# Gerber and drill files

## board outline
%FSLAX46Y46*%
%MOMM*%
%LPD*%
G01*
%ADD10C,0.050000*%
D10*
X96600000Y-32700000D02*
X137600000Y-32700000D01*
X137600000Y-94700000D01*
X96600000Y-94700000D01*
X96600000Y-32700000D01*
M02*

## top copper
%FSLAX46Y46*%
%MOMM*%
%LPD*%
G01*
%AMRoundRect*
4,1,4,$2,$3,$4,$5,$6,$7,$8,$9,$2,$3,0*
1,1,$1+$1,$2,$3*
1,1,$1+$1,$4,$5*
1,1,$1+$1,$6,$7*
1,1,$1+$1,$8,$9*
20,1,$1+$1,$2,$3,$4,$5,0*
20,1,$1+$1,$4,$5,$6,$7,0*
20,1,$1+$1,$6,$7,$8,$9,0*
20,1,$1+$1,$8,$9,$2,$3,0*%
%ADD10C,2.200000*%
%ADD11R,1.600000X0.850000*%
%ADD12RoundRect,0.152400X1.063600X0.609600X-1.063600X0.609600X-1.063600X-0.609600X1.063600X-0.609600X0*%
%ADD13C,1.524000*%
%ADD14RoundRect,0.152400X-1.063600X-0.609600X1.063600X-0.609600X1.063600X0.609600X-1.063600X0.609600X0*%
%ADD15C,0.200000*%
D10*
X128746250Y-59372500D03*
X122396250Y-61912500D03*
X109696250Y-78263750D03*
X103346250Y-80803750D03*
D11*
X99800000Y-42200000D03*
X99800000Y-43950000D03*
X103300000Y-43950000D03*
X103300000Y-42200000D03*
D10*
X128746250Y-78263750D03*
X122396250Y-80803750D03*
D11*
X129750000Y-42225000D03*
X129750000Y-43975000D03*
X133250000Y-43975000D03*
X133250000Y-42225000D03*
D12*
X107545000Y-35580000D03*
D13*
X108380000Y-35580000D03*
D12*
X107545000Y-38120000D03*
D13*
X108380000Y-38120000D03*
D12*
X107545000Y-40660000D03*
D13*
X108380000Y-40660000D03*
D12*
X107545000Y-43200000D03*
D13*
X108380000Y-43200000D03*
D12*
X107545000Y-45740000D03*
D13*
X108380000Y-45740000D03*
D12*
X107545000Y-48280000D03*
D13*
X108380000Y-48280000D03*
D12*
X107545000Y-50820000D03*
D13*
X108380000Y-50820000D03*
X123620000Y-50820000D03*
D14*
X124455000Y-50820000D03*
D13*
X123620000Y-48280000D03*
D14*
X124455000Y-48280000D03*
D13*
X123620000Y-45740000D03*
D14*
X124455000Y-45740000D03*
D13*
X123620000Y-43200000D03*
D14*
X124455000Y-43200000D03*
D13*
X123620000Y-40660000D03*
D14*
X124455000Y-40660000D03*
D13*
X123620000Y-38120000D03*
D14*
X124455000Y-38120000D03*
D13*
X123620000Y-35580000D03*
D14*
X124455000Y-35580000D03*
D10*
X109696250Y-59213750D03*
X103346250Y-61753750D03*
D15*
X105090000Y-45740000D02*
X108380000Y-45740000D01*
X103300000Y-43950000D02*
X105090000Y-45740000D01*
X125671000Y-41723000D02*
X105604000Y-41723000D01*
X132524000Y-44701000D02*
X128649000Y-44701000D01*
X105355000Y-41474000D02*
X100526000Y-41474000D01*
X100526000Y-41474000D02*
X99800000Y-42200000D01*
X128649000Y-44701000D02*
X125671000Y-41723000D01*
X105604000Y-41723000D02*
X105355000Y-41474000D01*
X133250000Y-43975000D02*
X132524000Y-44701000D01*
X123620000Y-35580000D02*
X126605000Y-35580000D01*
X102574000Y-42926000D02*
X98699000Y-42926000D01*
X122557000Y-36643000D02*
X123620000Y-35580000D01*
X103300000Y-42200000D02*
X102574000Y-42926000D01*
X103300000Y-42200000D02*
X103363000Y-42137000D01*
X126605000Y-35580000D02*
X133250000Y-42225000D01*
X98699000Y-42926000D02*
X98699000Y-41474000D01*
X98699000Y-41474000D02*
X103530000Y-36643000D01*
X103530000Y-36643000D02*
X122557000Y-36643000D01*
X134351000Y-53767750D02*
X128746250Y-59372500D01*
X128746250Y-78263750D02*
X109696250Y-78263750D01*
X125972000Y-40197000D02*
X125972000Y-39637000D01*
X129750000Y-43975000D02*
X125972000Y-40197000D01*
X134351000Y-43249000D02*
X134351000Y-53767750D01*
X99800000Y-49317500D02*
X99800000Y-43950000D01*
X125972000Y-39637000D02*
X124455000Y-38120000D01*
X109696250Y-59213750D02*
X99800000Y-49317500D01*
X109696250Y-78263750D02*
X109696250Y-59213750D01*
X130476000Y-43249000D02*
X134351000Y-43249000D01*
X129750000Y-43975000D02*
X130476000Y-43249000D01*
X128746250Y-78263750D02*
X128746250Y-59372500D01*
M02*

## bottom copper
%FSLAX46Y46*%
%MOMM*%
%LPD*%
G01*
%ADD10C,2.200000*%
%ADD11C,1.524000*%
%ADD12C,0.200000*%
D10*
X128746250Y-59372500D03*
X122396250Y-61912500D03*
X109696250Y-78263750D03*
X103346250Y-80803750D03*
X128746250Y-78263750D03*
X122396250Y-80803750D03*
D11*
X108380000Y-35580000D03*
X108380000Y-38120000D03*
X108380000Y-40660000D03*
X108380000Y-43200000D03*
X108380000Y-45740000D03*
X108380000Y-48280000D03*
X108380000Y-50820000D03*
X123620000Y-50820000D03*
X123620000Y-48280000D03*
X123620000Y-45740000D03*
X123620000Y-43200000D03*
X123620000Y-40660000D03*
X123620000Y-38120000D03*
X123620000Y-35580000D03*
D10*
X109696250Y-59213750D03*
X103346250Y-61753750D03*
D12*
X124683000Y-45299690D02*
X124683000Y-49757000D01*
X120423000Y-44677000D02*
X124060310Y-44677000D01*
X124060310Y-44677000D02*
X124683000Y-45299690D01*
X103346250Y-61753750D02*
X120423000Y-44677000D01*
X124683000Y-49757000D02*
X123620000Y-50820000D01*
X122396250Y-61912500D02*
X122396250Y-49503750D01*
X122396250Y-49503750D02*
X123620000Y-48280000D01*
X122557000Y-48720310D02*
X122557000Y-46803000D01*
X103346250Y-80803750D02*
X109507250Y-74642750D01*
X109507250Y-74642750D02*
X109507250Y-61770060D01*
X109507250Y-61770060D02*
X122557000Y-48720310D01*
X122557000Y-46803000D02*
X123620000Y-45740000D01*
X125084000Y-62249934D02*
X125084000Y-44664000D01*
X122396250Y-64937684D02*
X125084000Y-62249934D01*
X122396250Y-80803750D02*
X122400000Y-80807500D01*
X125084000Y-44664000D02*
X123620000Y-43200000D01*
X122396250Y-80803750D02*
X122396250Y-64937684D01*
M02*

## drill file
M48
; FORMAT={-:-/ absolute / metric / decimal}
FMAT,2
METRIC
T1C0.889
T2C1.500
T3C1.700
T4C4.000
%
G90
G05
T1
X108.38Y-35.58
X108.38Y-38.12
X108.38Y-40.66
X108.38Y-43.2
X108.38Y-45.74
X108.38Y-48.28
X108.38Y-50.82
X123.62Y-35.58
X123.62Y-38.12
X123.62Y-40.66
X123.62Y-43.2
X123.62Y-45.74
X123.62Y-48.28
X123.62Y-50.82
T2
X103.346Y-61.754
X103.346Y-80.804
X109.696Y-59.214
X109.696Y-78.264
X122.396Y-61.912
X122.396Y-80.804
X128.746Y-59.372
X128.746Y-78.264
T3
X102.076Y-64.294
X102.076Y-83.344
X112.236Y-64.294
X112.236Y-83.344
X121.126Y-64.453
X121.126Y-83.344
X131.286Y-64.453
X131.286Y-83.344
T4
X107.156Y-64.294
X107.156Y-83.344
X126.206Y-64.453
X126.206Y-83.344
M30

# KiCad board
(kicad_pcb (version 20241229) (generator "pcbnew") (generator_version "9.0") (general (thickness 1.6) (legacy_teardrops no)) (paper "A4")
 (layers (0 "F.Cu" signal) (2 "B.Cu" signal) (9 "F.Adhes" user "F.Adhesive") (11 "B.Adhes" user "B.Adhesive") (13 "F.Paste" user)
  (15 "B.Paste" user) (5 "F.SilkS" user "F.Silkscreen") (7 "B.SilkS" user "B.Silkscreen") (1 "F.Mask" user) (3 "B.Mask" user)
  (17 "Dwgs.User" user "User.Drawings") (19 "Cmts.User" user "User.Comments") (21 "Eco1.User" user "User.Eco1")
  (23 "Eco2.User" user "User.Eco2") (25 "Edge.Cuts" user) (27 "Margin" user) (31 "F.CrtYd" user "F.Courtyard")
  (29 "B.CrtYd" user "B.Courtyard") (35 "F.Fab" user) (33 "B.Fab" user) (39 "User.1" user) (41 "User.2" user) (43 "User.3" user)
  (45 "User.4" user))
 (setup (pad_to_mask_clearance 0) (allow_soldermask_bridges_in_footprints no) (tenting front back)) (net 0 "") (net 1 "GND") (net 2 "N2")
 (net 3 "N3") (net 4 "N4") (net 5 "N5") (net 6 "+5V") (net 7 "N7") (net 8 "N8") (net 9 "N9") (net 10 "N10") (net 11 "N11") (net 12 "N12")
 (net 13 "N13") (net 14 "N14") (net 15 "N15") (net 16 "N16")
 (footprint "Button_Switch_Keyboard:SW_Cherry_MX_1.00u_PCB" (layer "F.Cu") (at 128.74625 59.3725)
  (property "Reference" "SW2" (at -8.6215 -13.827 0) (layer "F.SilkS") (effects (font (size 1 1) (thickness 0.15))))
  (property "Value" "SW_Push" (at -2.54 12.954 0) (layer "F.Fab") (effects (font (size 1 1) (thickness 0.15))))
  (pad "" np_thru_hole circle (at -7.62 5.08) (size 1.7 1.7) (drill 1.7) (layers "*.Cu" "*.Mask"))
  (pad "" np_thru_hole circle (at -2.54 5.08) (size 4 4) (drill 4) (layers "*.Cu" "*.Mask"))
  (pad "" np_thru_hole circle (at 2.54 5.08) (size 1.7 1.7) (drill 1.7) (layers "*.Cu" "*.Mask"))
  (pad "1" thru_hole circle (at 0 0) (size 2.2 2.2) (drill 1.5) (layers "*.Cu" "*.Mask") (remove_unused_layers no) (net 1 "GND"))
  (pad "2" thru_hole circle (at -6.35 2.54) (size 2.2 2.2) (drill 1.5) (layers "*.Cu" "*.Mask") (remove_unused_layers no) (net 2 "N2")))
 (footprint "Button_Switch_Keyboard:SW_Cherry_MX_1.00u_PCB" (layer "F.Cu") (at 109.69625 78.26375)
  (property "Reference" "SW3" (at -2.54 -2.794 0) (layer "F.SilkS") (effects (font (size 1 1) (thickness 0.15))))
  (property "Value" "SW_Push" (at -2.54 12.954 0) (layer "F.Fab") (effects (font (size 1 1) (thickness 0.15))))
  (pad "" np_thru_hole circle (at -7.62 5.08) (size 1.7 1.7) (drill 1.7) (layers "*.Cu" "*.Mask"))
  (pad "" np_thru_hole circle (at -2.54 5.08) (size 4 4) (drill 4) (layers "*.Cu" "*.Mask"))
  (pad "" np_thru_hole circle (at 2.54 5.08) (size 1.7 1.7) (drill 1.7) (layers "*.Cu" "*.Mask"))
  (pad "1" thru_hole circle (at 0 0) (size 2.2 2.2) (drill 1.5) (layers "*.Cu" "*.Mask") (remove_unused_layers no) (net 1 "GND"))
  (pad "2" thru_hole circle (at -6.35 2.54) (size 2.2 2.2) (drill 1.5) (layers "*.Cu" "*.Mask") (remove_unused_layers no) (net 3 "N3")))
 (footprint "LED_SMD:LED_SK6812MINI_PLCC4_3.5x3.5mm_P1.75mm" (layer "F.Cu") (at 101.55 43.075)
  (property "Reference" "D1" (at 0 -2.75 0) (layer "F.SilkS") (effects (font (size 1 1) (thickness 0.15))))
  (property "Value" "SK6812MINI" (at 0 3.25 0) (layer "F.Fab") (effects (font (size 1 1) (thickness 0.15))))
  (pad "1" smd rect (at -1.75 -0.875) (size 1.6 0.85) (layers "F.Cu" "F.Mask" "F.Paste") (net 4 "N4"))
  (pad "2" smd rect (at -1.75 0.875) (size 1.6 0.85) (layers "F.Cu" "F.Mask" "F.Paste") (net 1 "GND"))
  (pad "3" smd rect (at 1.75 0.875) (size 1.6 0.85) (layers "F.Cu" "F.Mask" "F.Paste") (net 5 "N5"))
  (pad "4" smd rect (at 1.75 -0.875) (size 1.6 0.85) (layers "F.Cu" "F.Mask" "F.Paste") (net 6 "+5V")))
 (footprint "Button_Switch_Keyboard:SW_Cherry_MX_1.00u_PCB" (layer "F.Cu") (at 128.74625 78.26375)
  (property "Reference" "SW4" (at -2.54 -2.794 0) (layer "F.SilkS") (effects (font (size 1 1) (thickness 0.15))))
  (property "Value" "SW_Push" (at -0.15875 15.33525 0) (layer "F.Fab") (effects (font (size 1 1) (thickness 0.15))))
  (pad "" np_thru_hole circle (at -7.62 5.08) (size 1.7 1.7) (drill 1.7) (layers "*.Cu" "*.Mask"))
  (pad "" np_thru_hole circle (at -2.54 5.08) (size 4 4) (drill 4) (layers "*.Cu" "*.Mask"))
  (pad "" np_thru_hole circle (at 2.54 5.08) (size 1.7 1.7) (drill 1.7) (layers "*.Cu" "*.Mask"))
  (pad "1" thru_hole circle (at 0 0) (size 2.2 2.2) (drill 1.5) (layers "*.Cu" "*.Mask") (remove_unused_layers no) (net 1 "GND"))
  (pad "2" thru_hole circle (at -6.35 2.54) (size 2.2 2.2) (drill 1.5) (layers "*.Cu" "*.Mask") (remove_unused_layers no) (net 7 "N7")))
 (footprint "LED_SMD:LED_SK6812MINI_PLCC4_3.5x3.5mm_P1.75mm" (layer "F.Cu") (at 131.5 43.1)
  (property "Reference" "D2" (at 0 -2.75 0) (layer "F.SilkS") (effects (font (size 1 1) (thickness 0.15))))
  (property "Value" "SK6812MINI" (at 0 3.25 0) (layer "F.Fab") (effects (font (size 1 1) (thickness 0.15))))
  (pad "1" smd rect (at -1.75 -0.875) (size 1.6 0.85) (layers "F.Cu" "F.Mask" "F.Paste") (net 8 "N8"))
  (pad "2" smd rect (at -1.75 0.875) (size 1.6 0.85) (layers "F.Cu" "F.Mask" "F.Paste") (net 1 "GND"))
  (pad "3" smd rect (at 1.75 0.875) (size 1.6 0.85) (layers "F.Cu" "F.Mask" "F.Paste") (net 4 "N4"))
  (pad "4" smd rect (at 1.75 -0.875) (size 1.6 0.85) (layers "F.Cu" "F.Mask" "F.Paste") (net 6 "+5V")))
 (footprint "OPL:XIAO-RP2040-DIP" (layer "F.Cu") (at 116 43.2)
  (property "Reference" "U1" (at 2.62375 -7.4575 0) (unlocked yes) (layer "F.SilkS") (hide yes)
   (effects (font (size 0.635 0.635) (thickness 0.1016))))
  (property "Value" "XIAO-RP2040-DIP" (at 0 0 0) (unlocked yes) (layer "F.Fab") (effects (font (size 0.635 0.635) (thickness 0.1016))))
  (pad "1" smd roundrect (at -8.455 -7.62 180) (size 2.432 1.524) (layers "F.Cu" "F.Mask") (roundrect_rratio 0.1) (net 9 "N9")
   (thermal_bridge_angle 45))
  (pad "1" thru_hole circle (at -7.62 -7.62 180) (size 1.524 1.524) (drill 0.889) (layers "*.Cu" "*.Mask") (remove_unused_layers no)
   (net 9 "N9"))
  (pad "2" smd roundrect (at -8.455 -5.08 180) (size 2.432 1.524) (layers "F.Cu" "F.Mask") (roundrect_rratio 0.1) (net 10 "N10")
   (thermal_bridge_angle 45))
  (pad "2" thru_hole circle (at -7.62 -5.08 180) (size 1.524 1.524) (drill 0.889) (layers "*.Cu" "*.Mask") (remove_unused_layers no)
   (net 10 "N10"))
  (pad "3" smd roundrect (at -8.455 -2.54 180) (size 2.432 1.524) (layers "F.Cu" "F.Mask") (roundrect_rratio 0.1) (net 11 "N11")
   (thermal_bridge_angle 45))
  (pad "3" thru_hole circle (at -7.62 -2.54 180) (size 1.524 1.524) (drill 0.889) (layers "*.Cu" "*.Mask") (remove_unused_layers no)
   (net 11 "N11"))
  (pad "4" smd roundrect (at -8.455 0 180) (size 2.432 1.524) (layers "F.Cu" "F.Mask") (roundrect_rratio 0.1) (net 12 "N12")
   (thermal_bridge_angle 45))
  (pad "4" thru_hole circle (at -7.62 0 180) (size 1.524 1.524) (drill 0.889) (layers "*.Cu" "*.Mask") (remove_unused_layers no)
   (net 12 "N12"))
  (pad "5" smd roundrect (at -8.455 2.54 180) (size 2.432 1.524) (layers "F.Cu" "F.Mask") (roundrect_rratio 0.1) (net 5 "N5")
   (thermal_bridge_angle 45))
  (pad "5" thru_hole circle (at -7.62 2.54 180) (size 1.524 1.524) (drill 0.889) (layers "*.Cu" "*.Mask") (remove_unused_layers no)
   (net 5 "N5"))
  (pad "6" smd roundrect (at -8.455 5.08 180) (size 2.432 1.524) (layers "F.Cu" "F.Mask") (roundrect_rratio 0.1) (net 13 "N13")
   (thermal_bridge_angle 45))
  (pad "6" thru_hole circle (at -7.62 5.08 180) (size 1.524 1.524) (drill 0.889) (layers "*.Cu" "*.Mask") (remove_unused_layers no)
   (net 13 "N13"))
  (pad "7" smd roundrect (at -8.455 7.62 180) (size 2.432 1.524) (layers "F.Cu" "F.Mask") (roundrect_rratio 0.1) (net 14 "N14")
   (thermal_bridge_angle 45))
  (pad "7" thru_hole circle (at -7.62 7.62 180) (size 1.524 1.524) (drill 0.889) (layers "*.Cu" "*.Mask") (remove_unused_layers no)
   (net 14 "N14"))
  (pad "8" thru_hole circle (at 7.62 7.62) (size 1.524 1.524) (drill 0.889) (layers "*.Cu" "*.Mask") (remove_unused_layers no)
   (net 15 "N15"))
  (pad "8" smd roundrect (at 8.455 7.62) (size 2.432 1.524) (layers "F.Cu" "F.Mask") (roundrect_rratio 0.1) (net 15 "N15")
   (thermal_bridge_angle 45))
  (pad "9" thru_hole circle (at 7.62 5.08) (size 1.524 1.524) (drill 0.889) (layers "*.Cu" "*.Mask") (remove_unused_layers no) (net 2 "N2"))
  (pad "9" smd roundrect (at 8.455 5.08) (size 2.432 1.524) (layers "F.Cu" "F.Mask") (roundrect_rratio 0.1) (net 2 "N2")
   (thermal_bridge_angle 45))
  (pad "10" thru_hole circle (at 7.62 2.54) (size 1.524 1.524) (drill 0.889) (layers "*.Cu" "*.Mask") (remove_unused_layers no) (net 3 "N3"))
  (pad "10" smd roundrect (at 8.455 2.54) (size 2.432 1.524) (layers "F.Cu" "F.Mask") (roundrect_rratio 0.1) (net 3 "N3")
   (thermal_bridge_angle 45))
  (pad "11" thru_hole circle (at 7.62 0) (size 1.524 1.524) (drill 0.889) (layers "*.Cu" "*.Mask") (remove_unused_layers no) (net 7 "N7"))
  (pad "11" smd roundrect (at 8.455 0) (size 2.432 1.524) (layers "F.Cu" "F.Mask") (roundrect_rratio 0.1) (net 7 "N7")
   (thermal_bridge_angle 45))
  (pad "12" thru_hole circle (at 7.62 -2.54) (size 1.524 1.524) (drill 0.889) (layers "*.Cu" "*.Mask") (remove_unused_layers no)
   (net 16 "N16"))
  (pad "12" smd roundrect (at 8.455 -2.54) (size 2.432 1.524) (layers "F.Cu" "F.Mask") (roundrect_rratio 0.1) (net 16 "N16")
   (thermal_bridge_angle 45))
  (pad "13" thru_hole circle (at 7.62 -5.08) (size 1.524 1.524) (drill 0.889) (layers "*.Cu" "*.Mask") (remove_unused_layers no)
   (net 1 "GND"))
  (pad "13" smd roundrect (at 8.455 -5.08) (size 2.432 1.524) (layers "F.Cu" "F.Mask") (roundrect_rratio 0.1) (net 1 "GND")
   (thermal_bridge_angle 45))
  (pad "14" thru_hole circle (at 7.62 -7.62) (size 1.524 1.524) (drill 0.889) (layers "*.Cu" "*.Mask") (remove_unused_layers no)
   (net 6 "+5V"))
  (pad "14" smd roundrect (at 8.455 -7.62) (size 2.432 1.524) (layers "F.Cu" "F.Mask") (roundrect_rratio 0.1) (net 6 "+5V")
   (thermal_bridge_angle 45)))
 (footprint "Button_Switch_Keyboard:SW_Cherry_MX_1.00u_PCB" (layer "F.Cu") (at 109.69625 59.21375)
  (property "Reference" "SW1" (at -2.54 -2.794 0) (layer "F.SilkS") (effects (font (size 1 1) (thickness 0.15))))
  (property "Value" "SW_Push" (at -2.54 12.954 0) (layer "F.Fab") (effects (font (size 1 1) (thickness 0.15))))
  (pad "" np_thru_hole circle (at -7.62 5.08) (size 1.7 1.7) (drill 1.7) (layers "*.Cu" "*.Mask"))
  (pad "" np_thru_hole circle (at -2.54 5.08) (size 4 4) (drill 4) (layers "*.Cu" "*.Mask"))
  (pad "" np_thru_hole circle (at 2.54 5.08) (size 1.7 1.7) (drill 1.7) (layers "*.Cu" "*.Mask"))
  (pad "1" thru_hole circle (at 0 0) (size 2.2 2.2) (drill 1.5) (layers "*.Cu" "*.Mask") (remove_unused_layers no) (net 1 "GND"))
  (pad "2" thru_hole circle (at -6.35 2.54) (size 2.2 2.2) (drill 1.5) (layers "*.Cu" "*.Mask") (remove_unused_layers no) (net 15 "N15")))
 (gr_rect (start 96.6 32.7) (end 137.6 94.7) (stroke (width 0.05) (type default)) (fill no) (layer "Edge.Cuts"))
 (segment (start 105.09 45.74) (end 108.38 45.74) (width 0.2) (layer "F.Cu") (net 5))
 (segment (start 103.3 43.95) (end 105.09 45.74) (width 0.2) (layer "F.Cu") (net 5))
 (segment (start 125.671 41.723) (end 105.604 41.723) (width 0.2) (layer "F.Cu") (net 4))
 (segment (start 132.524 44.701) (end 128.649 44.701) (width 0.2) (layer "F.Cu") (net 4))
 (segment (start 105.355 41.474) (end 100.526 41.474) (width 0.2) (layer "F.Cu") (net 4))
 (segment (start 100.526 41.474) (end 99.8 42.2) (width 0.2) (layer "F.Cu") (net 4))
 (segment (start 128.649 44.701) (end 125.671 41.723) (width 0.2) (layer "F.Cu") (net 4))
 (segment (start 105.604 41.723) (end 105.355 41.474) (width 0.2) (layer "F.Cu") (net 4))
 (segment (start 133.25 43.975) (end 132.524 44.701) (width 0.2) (layer "F.Cu") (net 4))
 (segment (start 123.62 35.58) (end 126.605 35.58) (width 0.2) (layer "F.Cu") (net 6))
 (segment (start 102.574 42.926) (end 98.699 42.926) (width 0.2) (layer "F.Cu") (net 6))
 (segment (start 122.557 36.643) (end 123.62 35.58) (width 0.2) (layer "F.Cu") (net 6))
 (segment (start 103.3 42.2) (end 102.574 42.926) (width 0.2) (layer "F.Cu") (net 6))
 (segment (start 103.3 42.2) (end 103.363 42.137) (width 0.2) (layer "F.Cu") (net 6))
 (segment (start 126.605 35.58) (end 133.25 42.225) (width 0.2) (layer "F.Cu") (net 6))
 (segment (start 98.699 42.926) (end 98.699 41.474) (width 0.2) (layer "F.Cu") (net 6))
 (segment (start 98.699 41.474) (end 103.53 36.643) (width 0.2) (layer "F.Cu") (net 6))
 (segment (start 103.53 36.643) (end 122.557 36.643) (width 0.2) (layer "F.Cu") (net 6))
 (segment (start 134.351 53.76775) (end 128.74625 59.3725) (width 0.2) (layer "F.Cu") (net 1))
 (segment (start 128.74625 78.26375) (end 109.69625 78.26375) (width 0.2) (layer "F.Cu") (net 1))
 (segment (start 125.972 40.197) (end 125.972 39.637) (width 0.2) (layer "F.Cu") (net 1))
 (segment (start 129.75 43.975) (end 125.972 40.197) (width 0.2) (layer "F.Cu") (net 1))
 (segment (start 134.351 43.249) (end 134.351 53.76775) (width 0.2) (layer "F.Cu") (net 1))
 (segment (start 99.8 49.3175) (end 99.8 43.95) (width 0.2) (layer "F.Cu") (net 1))
 (segment (start 125.972 39.637) (end 124.455 38.12) (width 0.2) (layer "F.Cu") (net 1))
 (segment (start 109.69625 59.21375) (end 99.8 49.3175) (width 0.2) (layer "F.Cu") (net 1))
 (segment (start 109.69625 78.26375) (end 109.69625 59.21375) (width 0.2) (layer "F.Cu") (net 1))
 (segment (start 130.476 43.249) (end 134.351 43.249) (width 0.2) (layer "F.Cu") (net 1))
 (segment (start 129.75 43.975) (end 130.476 43.249) (width 0.2) (layer "F.Cu") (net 1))
 (segment (start 128.74625 78.26375) (end 128.74625 59.3725) (width 0.2) (layer "F.Cu") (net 1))
 (segment (start 124.683 45.29969) (end 124.683 49.757) (width 0.2) (layer "B.Cu") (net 15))
 (segment (start 120.423 44.677) (end 124.06031 44.677) (width 0.2) (layer "B.Cu") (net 15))
 (segment (start 124.06031 44.677) (end 124.683 45.29969) (width 0.2) (layer "B.Cu") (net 15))
 (segment (start 103.34625 61.75375) (end 120.423 44.677) (width 0.2) (layer "B.Cu") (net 15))
 (segment (start 124.683 49.757) (end 123.62 50.82) (width 0.2) (layer "B.Cu") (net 15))
 (segment (start 122.39625 61.9125) (end 122.39625 49.50375) (width 0.2) (layer "B.Cu") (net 2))
 (segment (start 122.39625 49.50375) (end 123.62 48.28) (width 0.2) (layer "B.Cu") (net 2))
 (segment (start 122.557 48.72031) (end 122.557 46.803) (width 0.2) (layer "B.Cu") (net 3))
 (segment (start 103.34625 80.80375) (end 109.50725 74.64275) (width 0.2) (layer "B.Cu") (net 3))
 (segment (start 109.50725 74.64275) (end 109.50725 61.77006) (width 0.2) (layer "B.Cu") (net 3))
 (segment (start 109.50725 61.77006) (end 122.557 48.72031) (width 0.2) (layer "B.Cu") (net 3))
 (segment (start 122.557 46.803) (end 123.62 45.74) (width 0.2) (layer "B.Cu") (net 3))
 (segment (start 125.084 62.249934) (end 125.084 44.664) (width 0.2) (layer "B.Cu") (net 7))
 (segment (start 122.39625 64.937684) (end 125.084 62.249934) (width 0.2) (layer "B.Cu") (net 7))
 (segment (start 122.39625 80.80375) (end 122.4 80.8075) (width 0.2) (layer "B.Cu") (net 7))
 (segment (start 125.084 44.664) (end 123.62 43.2) (width 0.2) (layer "B.Cu") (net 7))
 (segment (start 122.39625 80.80375) (end 122.39625 64.937684) (width 0.2) (layer "B.Cu") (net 7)))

